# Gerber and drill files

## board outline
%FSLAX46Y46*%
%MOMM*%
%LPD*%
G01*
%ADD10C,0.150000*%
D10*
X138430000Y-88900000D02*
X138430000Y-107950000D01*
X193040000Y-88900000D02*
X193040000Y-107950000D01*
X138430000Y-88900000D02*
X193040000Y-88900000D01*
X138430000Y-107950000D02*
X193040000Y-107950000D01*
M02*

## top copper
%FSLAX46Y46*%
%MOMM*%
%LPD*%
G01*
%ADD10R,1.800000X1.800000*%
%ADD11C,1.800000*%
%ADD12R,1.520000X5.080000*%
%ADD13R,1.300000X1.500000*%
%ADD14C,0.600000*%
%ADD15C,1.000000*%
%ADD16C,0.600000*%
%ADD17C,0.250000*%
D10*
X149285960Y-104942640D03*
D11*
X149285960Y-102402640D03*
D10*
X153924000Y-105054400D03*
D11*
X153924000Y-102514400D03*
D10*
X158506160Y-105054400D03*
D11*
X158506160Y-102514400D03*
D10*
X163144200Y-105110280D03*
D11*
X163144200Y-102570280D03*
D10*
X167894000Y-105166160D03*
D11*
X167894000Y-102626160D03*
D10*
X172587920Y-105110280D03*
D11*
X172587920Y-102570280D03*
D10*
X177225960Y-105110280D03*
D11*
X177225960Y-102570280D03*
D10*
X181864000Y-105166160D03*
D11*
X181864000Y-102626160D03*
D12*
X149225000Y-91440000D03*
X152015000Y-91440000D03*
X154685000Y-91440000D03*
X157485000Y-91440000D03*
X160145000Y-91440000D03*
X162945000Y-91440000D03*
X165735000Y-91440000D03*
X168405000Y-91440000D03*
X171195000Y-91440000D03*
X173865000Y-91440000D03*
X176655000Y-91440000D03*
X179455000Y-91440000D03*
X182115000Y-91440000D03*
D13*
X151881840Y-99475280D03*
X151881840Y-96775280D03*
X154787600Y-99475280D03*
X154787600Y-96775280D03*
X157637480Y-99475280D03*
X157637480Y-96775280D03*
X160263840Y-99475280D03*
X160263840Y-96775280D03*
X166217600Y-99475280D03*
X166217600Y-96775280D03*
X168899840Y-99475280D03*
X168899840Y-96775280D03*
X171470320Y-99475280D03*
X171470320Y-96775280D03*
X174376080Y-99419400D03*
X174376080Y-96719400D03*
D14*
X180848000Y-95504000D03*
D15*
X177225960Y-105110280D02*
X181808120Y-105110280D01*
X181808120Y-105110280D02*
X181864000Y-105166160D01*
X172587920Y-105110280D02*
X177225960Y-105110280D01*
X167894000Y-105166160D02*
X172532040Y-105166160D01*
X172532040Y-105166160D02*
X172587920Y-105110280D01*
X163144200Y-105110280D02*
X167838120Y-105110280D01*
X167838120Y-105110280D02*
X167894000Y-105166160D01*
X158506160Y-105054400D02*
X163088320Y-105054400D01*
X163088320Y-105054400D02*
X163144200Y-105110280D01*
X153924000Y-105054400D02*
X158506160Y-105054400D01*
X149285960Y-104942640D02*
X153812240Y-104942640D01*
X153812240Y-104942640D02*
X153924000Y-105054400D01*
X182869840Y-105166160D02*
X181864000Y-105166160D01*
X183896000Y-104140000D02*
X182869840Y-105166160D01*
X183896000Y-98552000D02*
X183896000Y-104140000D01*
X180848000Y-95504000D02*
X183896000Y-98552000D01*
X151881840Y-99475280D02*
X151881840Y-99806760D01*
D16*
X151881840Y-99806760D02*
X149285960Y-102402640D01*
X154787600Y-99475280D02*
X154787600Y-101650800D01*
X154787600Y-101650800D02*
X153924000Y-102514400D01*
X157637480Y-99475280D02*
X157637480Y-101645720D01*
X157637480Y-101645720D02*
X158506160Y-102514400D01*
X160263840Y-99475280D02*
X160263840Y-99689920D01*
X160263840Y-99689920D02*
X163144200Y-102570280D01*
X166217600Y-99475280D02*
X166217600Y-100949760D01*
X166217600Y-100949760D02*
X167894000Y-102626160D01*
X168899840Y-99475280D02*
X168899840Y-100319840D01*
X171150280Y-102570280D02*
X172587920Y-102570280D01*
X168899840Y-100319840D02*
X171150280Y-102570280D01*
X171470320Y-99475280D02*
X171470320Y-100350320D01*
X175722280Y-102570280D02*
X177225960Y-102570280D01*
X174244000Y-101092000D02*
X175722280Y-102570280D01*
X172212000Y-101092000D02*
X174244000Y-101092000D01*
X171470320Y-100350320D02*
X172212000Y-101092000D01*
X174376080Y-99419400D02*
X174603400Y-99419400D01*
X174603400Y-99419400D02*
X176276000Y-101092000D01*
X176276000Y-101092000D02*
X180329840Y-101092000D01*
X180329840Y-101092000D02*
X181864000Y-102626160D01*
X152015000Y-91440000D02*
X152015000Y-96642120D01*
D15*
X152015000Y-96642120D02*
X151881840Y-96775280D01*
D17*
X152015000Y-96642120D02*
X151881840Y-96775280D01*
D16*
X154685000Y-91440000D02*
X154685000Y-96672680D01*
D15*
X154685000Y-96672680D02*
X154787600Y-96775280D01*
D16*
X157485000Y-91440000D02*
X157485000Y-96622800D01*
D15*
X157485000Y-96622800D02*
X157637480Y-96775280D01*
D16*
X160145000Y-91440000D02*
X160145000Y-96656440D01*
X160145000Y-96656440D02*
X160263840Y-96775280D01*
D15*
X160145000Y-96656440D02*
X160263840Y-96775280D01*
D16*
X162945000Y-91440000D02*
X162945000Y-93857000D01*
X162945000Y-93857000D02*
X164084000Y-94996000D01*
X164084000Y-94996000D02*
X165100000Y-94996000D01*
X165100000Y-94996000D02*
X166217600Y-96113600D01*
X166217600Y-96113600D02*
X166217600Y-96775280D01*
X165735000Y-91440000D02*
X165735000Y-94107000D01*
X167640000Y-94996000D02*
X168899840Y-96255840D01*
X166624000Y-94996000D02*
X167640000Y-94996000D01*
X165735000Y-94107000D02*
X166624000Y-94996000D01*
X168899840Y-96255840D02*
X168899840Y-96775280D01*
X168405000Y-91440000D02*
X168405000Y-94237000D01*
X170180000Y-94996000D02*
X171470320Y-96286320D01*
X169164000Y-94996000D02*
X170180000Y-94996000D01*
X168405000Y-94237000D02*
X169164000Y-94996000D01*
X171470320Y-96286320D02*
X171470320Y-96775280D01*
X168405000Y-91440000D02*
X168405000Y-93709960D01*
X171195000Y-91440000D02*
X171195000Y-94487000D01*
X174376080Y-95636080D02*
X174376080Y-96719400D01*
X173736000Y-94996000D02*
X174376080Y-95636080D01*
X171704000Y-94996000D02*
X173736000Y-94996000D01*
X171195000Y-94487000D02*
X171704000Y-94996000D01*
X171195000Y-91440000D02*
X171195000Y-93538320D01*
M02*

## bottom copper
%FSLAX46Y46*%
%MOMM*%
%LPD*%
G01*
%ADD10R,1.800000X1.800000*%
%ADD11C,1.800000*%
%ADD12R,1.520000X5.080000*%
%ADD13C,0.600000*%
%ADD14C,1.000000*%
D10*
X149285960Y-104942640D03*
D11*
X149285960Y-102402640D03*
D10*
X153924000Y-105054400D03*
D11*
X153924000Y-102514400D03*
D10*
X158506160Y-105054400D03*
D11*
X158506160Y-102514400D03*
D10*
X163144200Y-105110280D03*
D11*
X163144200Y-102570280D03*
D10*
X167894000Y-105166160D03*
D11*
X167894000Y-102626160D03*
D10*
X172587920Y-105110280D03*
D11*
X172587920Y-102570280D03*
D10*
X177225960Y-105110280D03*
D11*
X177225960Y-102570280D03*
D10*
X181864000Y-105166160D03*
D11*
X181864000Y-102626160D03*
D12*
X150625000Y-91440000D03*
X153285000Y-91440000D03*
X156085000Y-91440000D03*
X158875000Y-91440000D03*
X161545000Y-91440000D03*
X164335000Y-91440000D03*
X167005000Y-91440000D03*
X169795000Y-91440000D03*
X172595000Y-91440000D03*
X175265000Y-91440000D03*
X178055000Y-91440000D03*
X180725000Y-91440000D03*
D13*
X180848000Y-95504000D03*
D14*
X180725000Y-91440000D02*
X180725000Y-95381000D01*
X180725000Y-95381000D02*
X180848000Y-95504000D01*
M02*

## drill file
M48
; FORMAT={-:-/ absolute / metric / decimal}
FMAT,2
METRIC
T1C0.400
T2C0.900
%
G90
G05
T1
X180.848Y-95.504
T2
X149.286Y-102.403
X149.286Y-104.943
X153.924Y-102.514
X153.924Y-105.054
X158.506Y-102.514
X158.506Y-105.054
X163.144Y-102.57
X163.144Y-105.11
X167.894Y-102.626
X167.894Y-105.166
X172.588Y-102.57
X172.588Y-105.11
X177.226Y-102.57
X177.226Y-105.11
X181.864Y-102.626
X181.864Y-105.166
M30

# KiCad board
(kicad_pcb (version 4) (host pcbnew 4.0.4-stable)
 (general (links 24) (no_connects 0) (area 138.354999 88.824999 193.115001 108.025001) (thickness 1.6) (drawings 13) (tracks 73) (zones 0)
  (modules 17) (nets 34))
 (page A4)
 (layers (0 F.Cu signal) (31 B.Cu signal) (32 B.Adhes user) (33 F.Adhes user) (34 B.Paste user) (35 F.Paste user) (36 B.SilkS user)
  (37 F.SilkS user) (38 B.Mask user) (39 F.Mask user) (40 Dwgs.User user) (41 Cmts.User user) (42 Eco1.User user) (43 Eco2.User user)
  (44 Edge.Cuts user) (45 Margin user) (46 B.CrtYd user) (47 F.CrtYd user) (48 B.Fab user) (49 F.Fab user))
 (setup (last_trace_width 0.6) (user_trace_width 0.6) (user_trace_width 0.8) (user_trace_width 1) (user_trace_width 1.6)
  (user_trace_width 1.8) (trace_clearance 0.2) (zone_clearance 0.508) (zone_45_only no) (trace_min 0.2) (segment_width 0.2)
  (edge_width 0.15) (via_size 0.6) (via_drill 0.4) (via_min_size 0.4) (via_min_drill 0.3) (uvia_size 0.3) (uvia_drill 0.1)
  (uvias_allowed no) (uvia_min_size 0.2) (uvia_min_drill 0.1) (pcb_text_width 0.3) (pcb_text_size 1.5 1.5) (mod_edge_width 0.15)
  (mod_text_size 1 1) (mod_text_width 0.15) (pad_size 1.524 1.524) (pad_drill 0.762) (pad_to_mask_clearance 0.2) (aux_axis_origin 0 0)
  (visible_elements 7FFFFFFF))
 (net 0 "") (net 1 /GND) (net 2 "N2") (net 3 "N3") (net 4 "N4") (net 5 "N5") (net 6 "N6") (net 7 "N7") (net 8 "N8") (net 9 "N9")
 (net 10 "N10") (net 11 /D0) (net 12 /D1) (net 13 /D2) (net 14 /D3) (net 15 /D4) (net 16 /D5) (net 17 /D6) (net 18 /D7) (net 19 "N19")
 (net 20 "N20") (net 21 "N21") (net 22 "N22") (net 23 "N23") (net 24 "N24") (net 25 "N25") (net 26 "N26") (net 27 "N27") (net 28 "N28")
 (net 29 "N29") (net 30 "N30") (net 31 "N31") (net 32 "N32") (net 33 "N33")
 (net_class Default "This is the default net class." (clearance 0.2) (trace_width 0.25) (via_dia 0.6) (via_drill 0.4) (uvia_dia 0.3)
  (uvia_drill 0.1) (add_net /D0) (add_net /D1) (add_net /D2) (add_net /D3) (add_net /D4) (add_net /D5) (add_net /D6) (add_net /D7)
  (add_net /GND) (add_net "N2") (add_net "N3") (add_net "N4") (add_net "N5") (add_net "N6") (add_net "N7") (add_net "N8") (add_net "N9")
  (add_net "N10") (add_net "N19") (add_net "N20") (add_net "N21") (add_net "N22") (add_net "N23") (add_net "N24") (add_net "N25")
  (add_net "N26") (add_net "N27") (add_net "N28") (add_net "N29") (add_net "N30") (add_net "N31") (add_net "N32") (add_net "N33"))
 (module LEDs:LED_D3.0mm (layer F.Cu) (at 149.28596 104.94264 90)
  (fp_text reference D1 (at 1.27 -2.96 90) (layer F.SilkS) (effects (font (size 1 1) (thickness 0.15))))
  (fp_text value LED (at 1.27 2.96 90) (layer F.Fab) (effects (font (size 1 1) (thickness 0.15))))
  (pad 1 thru_hole rect (at 0 0 90) (size 1.8 1.8) (drill 0.9) (layers *.Cu *.Mask) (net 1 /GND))
  (pad 2 thru_hole circle (at 2.54 0 90) (size 1.8 1.8) (drill 0.9) (layers *.Cu *.Mask) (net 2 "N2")))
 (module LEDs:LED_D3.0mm (layer F.Cu) (at 153.924 105.0544 90)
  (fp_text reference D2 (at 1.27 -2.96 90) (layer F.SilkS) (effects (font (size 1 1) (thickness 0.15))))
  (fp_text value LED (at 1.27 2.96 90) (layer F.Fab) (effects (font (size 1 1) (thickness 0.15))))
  (pad 1 thru_hole rect (at 0 0 90) (size 1.8 1.8) (drill 0.9) (layers *.Cu *.Mask) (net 1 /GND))
  (pad 2 thru_hole circle (at 2.54 0 90) (size 1.8 1.8) (drill 0.9) (layers *.Cu *.Mask) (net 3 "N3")))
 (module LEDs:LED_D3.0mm (layer F.Cu) (at 158.50616 105.0544 90)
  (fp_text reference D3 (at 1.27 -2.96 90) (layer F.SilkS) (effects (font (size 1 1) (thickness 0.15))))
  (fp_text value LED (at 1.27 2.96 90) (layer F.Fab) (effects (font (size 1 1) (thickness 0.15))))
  (pad 1 thru_hole rect (at 0 0 90) (size 1.8 1.8) (drill 0.9) (layers *.Cu *.Mask) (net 1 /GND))
  (pad 2 thru_hole circle (at 2.54 0 90) (size 1.8 1.8) (drill 0.9) (layers *.Cu *.Mask) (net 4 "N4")))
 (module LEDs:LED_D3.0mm (layer F.Cu) (at 163.1442 105.11028 90)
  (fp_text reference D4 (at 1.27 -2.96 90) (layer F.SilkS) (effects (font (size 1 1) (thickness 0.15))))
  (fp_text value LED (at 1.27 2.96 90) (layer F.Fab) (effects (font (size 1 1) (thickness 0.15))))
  (pad 1 thru_hole rect (at 0 0 90) (size 1.8 1.8) (drill 0.9) (layers *.Cu *.Mask) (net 1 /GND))
  (pad 2 thru_hole circle (at 2.54 0 90) (size 1.8 1.8) (drill 0.9) (layers *.Cu *.Mask) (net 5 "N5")))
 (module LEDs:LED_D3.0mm (layer F.Cu) (at 167.894 105.16616 90)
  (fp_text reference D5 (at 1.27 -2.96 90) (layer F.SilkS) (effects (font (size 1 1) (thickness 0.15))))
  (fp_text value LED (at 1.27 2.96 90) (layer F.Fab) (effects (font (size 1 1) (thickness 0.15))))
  (pad 1 thru_hole rect (at 0 0 90) (size 1.8 1.8) (drill 0.9) (layers *.Cu *.Mask) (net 1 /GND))
  (pad 2 thru_hole circle (at 2.54 0 90) (size 1.8 1.8) (drill 0.9) (layers *.Cu *.Mask) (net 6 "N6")))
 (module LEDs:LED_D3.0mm (layer F.Cu) (at 172.58792 105.11028 90)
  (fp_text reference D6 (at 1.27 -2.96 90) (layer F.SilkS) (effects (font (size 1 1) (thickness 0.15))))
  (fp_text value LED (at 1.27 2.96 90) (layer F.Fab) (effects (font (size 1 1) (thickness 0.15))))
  (pad 1 thru_hole rect (at 0 0 90) (size 1.8 1.8) (drill 0.9) (layers *.Cu *.Mask) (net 1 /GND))
  (pad 2 thru_hole circle (at 2.54 0 90) (size 1.8 1.8) (drill 0.9) (layers *.Cu *.Mask) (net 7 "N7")))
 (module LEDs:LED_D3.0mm (layer F.Cu) (at 177.22596 105.11028 90)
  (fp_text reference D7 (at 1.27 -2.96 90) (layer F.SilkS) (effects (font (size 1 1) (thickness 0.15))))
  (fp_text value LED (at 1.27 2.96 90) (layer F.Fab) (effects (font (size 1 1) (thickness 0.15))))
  (pad 1 thru_hole rect (at 0 0 90) (size 1.8 1.8) (drill 0.9) (layers *.Cu *.Mask) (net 1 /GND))
  (pad 2 thru_hole circle (at 2.54 0 90) (size 1.8 1.8) (drill 0.9) (layers *.Cu *.Mask) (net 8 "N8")))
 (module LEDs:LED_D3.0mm (layer F.Cu) (at 181.864 105.16616 90)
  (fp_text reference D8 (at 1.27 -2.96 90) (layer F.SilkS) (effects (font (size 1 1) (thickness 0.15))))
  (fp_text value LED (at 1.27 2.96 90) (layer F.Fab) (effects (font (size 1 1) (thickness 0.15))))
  (pad 1 thru_hole rect (at 0 0 90) (size 1.8 1.8) (drill 0.9) (layers *.Cu *.Mask) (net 1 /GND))
  (pad 2 thru_hole circle (at 2.54 0 90) (size 1.8 1.8) (drill 0.9) (layers *.Cu *.Mask) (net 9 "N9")))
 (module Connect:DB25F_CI (layer F.Cu) (at 149.225 91.44)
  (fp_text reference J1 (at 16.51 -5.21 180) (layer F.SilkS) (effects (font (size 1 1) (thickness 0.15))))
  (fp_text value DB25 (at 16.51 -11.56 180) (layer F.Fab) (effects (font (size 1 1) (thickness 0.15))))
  (pad 1 connect rect (at 0 0 90) (size 5.08 1.52) (layers F.Cu F.Mask) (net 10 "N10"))
  (pad 2 connect rect (at 2.79 0 90) (size 5.08 1.52) (layers F.Cu F.Mask) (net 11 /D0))
  (pad 3 connect rect (at 5.46 0 90) (size 5.08 1.52) (layers F.Cu F.Mask) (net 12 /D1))
  (pad 4 connect rect (at 8.26 0 90) (size 5.08 1.52) (layers F.Cu F.Mask) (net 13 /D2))
  (pad 5 connect rect (at 10.92 0 90) (size 5.08 1.52) (layers F.Cu F.Mask) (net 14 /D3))
  (pad 6 connect rect (at 13.72 0 90) (size 5.08 1.52) (layers F.Cu F.Mask) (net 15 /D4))
  (pad 7 connect rect (at 16.51 0 90) (size 5.08 1.52) (layers F.Cu F.Mask) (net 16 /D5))
  (pad 8 connect rect (at 19.18 0 90) (size 5.08 1.52) (layers F.Cu F.Mask) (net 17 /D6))
  (pad 9 connect rect (at 21.97 0 90) (size 5.08 1.52) (layers F.Cu F.Mask) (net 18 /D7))
  (pad 10 connect rect (at 24.64 0 90) (size 5.08 1.52) (layers F.Cu F.Mask) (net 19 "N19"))
  (pad 11 connect rect (at 27.43 0 90) (size 5.08 1.52) (layers F.Cu F.Mask) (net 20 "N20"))
  (pad 12 connect rect (at 30.23 0 90) (size 5.08 1.52) (layers F.Cu F.Mask) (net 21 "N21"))
  (pad 13 connect rect (at 32.89 0 90) (size 5.08 1.52) (layers F.Cu F.Mask) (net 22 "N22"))
  (pad 14 connect rect (at 1.4 0 90) (size 5.08 1.52) (layers B.Cu B.Mask) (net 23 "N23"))
  (pad 15 connect rect (at 4.06 0 90) (size 5.08 1.52) (layers B.Cu B.Mask) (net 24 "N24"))
  (pad 16 connect rect (at 6.86 0 90) (size 5.08 1.52) (layers B.Cu B.Mask) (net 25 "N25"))
  (pad 17 connect rect (at 9.65 0 90) (size 5.08 1.52) (layers B.Cu B.Mask) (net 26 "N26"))
  (pad 18 connect rect (at 12.32 0 90) (size 5.08 1.52) (layers B.Cu B.Mask) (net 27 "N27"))
  (pad 19 connect rect (at 15.11 0 90) (size 5.08 1.52) (layers B.Cu B.Mask) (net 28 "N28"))
  (pad 20 connect rect (at 17.78 0 90) (size 5.08 1.52) (layers B.Cu B.Mask) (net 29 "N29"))
  (pad 21 connect rect (at 20.57 0 90) (size 5.08 1.52) (layers B.Cu B.Mask) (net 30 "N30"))
  (pad 22 connect rect (at 23.37 0 90) (size 5.08 1.52) (layers B.Cu B.Mask) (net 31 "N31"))
  (pad 23 connect rect (at 26.04 0 90) (size 5.08 1.52) (layers B.Cu B.Mask) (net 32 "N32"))
  (pad 24 connect rect (at 28.83 0 90) (size 5.08 1.52) (layers B.Cu B.Mask) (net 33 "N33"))
  (pad 25 connect rect (at 31.5 0 90) (size 5.08 1.52) (layers B.Cu B.Mask) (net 1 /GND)))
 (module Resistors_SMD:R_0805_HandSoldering (layer F.Cu) (at 151.88184 98.12528 90)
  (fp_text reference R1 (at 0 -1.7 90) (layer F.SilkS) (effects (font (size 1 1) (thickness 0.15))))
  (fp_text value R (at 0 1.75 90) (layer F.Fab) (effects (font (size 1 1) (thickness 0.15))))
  (pad 1 smd rect (at -1.35 0 90) (size 1.5 1.3) (layers F.Cu F.Paste F.Mask) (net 2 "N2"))
  (pad 2 smd rect (at 1.35 0 90) (size 1.5 1.3) (layers F.Cu F.Paste F.Mask) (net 11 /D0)))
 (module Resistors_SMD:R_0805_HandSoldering (layer F.Cu) (at 154.7876 98.12528 90)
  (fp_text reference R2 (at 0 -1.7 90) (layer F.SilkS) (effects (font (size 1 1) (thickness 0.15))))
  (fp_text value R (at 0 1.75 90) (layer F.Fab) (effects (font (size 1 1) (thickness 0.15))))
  (pad 1 smd rect (at -1.35 0 90) (size 1.5 1.3) (layers F.Cu F.Paste F.Mask) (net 3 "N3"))
  (pad 2 smd rect (at 1.35 0 90) (size 1.5 1.3) (layers F.Cu F.Paste F.Mask) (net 12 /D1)))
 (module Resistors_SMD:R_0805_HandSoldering (layer F.Cu) (at 157.63748 98.12528 90)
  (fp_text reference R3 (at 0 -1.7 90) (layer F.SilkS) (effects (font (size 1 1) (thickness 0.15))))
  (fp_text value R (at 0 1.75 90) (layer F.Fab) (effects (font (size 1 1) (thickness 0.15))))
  (pad 1 smd rect (at -1.35 0 90) (size 1.5 1.3) (layers F.Cu F.Paste F.Mask) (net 4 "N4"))
  (pad 2 smd rect (at 1.35 0 90) (size 1.5 1.3) (layers F.Cu F.Paste F.Mask) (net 13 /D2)))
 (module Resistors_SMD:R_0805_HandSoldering (layer F.Cu) (at 160.26384 98.12528 90)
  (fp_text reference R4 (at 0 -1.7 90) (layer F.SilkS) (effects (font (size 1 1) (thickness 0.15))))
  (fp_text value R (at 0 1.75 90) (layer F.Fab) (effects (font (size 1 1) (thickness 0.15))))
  (pad 1 smd rect (at -1.35 0 90) (size 1.5 1.3) (layers F.Cu F.Paste F.Mask) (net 5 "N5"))
  (pad 2 smd rect (at 1.35 0 90) (size 1.5 1.3) (layers F.Cu F.Paste F.Mask) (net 14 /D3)))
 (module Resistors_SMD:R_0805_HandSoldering (layer F.Cu) (at 166.2176 98.12528 90)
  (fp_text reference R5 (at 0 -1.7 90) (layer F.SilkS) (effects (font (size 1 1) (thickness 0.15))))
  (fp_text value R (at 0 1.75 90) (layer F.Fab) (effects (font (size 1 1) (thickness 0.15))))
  (pad 1 smd rect (at -1.35 0 90) (size 1.5 1.3) (layers F.Cu F.Paste F.Mask) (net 6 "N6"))
  (pad 2 smd rect (at 1.35 0 90) (size 1.5 1.3) (layers F.Cu F.Paste F.Mask) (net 15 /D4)))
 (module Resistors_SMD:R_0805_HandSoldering (layer F.Cu) (at 168.89984 98.12528 90)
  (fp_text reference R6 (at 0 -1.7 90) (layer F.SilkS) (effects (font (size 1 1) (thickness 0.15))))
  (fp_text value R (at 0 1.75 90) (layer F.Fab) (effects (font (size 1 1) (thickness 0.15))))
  (pad 1 smd rect (at -1.35 0 90) (size 1.5 1.3) (layers F.Cu F.Paste F.Mask) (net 7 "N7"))
  (pad 2 smd rect (at 1.35 0 90) (size 1.5 1.3) (layers F.Cu F.Paste F.Mask) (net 16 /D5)))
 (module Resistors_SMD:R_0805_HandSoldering (layer F.Cu) (at 171.47032 98.12528 90)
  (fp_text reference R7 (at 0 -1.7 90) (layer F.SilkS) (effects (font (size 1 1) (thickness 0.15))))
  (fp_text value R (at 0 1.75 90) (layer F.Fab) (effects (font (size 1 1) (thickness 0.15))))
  (pad 1 smd rect (at -1.35 0 90) (size 1.5 1.3) (layers F.Cu F.Paste F.Mask) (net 8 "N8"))
  (pad 2 smd rect (at 1.35 0 90) (size 1.5 1.3) (layers F.Cu F.Paste F.Mask) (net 17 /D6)))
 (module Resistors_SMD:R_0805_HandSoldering (layer F.Cu) (at 174.37608 98.0694 90)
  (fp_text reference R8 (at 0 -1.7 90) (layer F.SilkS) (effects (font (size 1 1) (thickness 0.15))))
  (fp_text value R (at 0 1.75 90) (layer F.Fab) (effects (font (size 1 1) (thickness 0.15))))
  (pad 1 smd rect (at -1.35 0 90) (size 1.5 1.3) (layers F.Cu F.Paste F.Mask) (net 9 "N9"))
  (pad 2 smd rect (at 1.35 0 90) (size 1.5 1.3) (layers F.Cu F.Paste F.Mask) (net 18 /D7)))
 (gr_line (start 138.43 88.9) (end 138.43 107.95) (angle 90) (layer Edge.Cuts) (width 0.15))
 (gr_line (start 193.04 88.9) (end 193.04 107.95) (angle 90) (layer Edge.Cuts) (width 0.15))
 (gr_line (start 138.43 88.9) (end 193.04 88.9) (angle 90) (layer Edge.Cuts) (width 0.15))
 (gr_line (start 138.43 107.95) (end 193.04 107.95) (angle 90) (layer Edge.Cuts) (width 0.15))
 (segment (start 177.22596 105.11028) (end 181.80812 105.11028) (width 1) (layer F.Cu) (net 1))
 (segment (start 181.80812 105.11028) (end 181.864 105.16616) (width 1) (layer F.Cu) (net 1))
 (segment (start 172.58792 105.11028) (end 177.22596 105.11028) (width 1) (layer F.Cu) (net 1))
 (segment (start 167.894 105.16616) (end 172.53204 105.16616) (width 1) (layer F.Cu) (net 1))
 (segment (start 172.53204 105.16616) (end 172.58792 105.11028) (width 1) (layer F.Cu) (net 1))
 (segment (start 163.1442 105.11028) (end 167.83812 105.11028) (width 1) (layer F.Cu) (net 1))
 (segment (start 167.83812 105.11028) (end 167.894 105.16616) (width 1) (layer F.Cu) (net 1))
 (segment (start 158.50616 105.0544) (end 163.08832 105.0544) (width 1) (layer F.Cu) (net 1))
 (segment (start 163.08832 105.0544) (end 163.1442 105.11028) (width 1) (layer F.Cu) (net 1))
 (segment (start 153.924 105.0544) (end 158.50616 105.0544) (width 1) (layer F.Cu) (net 1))
 (segment (start 149.28596 104.94264) (end 153.81224 104.94264) (width 1) (layer F.Cu) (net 1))
 (segment (start 153.81224 104.94264) (end 153.924 105.0544) (width 1) (layer F.Cu) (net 1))
 (segment (start 180.725 91.44) (end 180.725 95.381) (width 1) (layer B.Cu) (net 1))
 (segment (start 182.86984 105.16616) (end 181.864 105.16616) (width 1) (layer F.Cu) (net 1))
 (segment (start 183.896 104.14) (end 182.86984 105.16616) (width 1) (layer F.Cu) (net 1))
 (segment (start 183.896 98.552) (end 183.896 104.14) (width 1) (layer F.Cu) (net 1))
 (segment (start 180.848 95.504) (end 183.896 98.552) (width 1) (layer F.Cu) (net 1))
 (via (at 180.848 95.504) (size 0.6) (drill 0.4) (layers F.Cu B.Cu) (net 1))
 (segment (start 180.725 95.381) (end 180.848 95.504) (width 1) (layer B.Cu) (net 1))
 (segment (start 151.88184 99.47528) (end 151.88184 99.80676) (width 1) (layer F.Cu) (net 2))
 (segment (start 151.88184 99.80676) (end 149.28596 102.40264) (width 0.6) (layer F.Cu) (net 2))
 (segment (start 154.7876 99.47528) (end 154.7876 101.6508) (width 0.6) (layer F.Cu) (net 3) (status 400000))
 (segment (start 154.7876 101.6508) (end 153.924 102.5144) (width 0.6) (layer F.Cu) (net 3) (status 800000))
 (segment (start 157.63748 99.47528) (end 157.63748 101.64572) (width 0.6) (layer F.Cu) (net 4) (status 400000))
 (segment (start 157.63748 101.64572) (end 158.50616 102.5144) (width 0.6) (layer F.Cu) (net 4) (status 800000))
 (segment (start 160.26384 99.47528) (end 160.26384 99.68992) (width 0.6) (layer F.Cu) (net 5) (status C00000))
 (segment (start 160.26384 99.68992) (end 163.1442 102.57028) (width 0.6) (layer F.Cu) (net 5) (status C00000))
 (segment (start 166.2176 99.47528) (end 166.2176 100.94976) (width 0.6) (layer F.Cu) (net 6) (status 400000))
 (segment (start 166.2176 100.94976) (end 167.894 102.62616) (width 0.6) (layer F.Cu) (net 6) (status 800000))
 (segment (start 168.89984 99.47528) (end 168.89984 100.31984) (width 0.6) (layer F.Cu) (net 7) (status 400000))
 (segment (start 171.15028 102.57028) (end 172.58792 102.57028) (width 0.6) (layer F.Cu) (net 7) (status 800000))
 (segment (start 168.89984 100.31984) (end 171.15028 102.57028) (width 0.6) (layer F.Cu) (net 7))
 (segment (start 171.47032 99.47528) (end 171.47032 100.35032) (width 0.6) (layer F.Cu) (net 8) (status 400000))
 (segment (start 175.72228 102.57028) (end 177.22596 102.57028) (width 0.6) (layer F.Cu) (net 8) (status 800000))
 (segment (start 174.244 101.092) (end 175.72228 102.57028) (width 0.6) (layer F.Cu) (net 8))
 (segment (start 172.212 101.092) (end 174.244 101.092) (width 0.6) (layer F.Cu) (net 8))
 (segment (start 171.47032 100.35032) (end 172.212 101.092) (width 0.6) (layer F.Cu) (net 8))
 (segment (start 174.37608 99.4194) (end 174.6034 99.4194) (width 0.6) (layer F.Cu) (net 9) (status C00000))
 (segment (start 174.6034 99.4194) (end 176.276 101.092) (width 0.6) (layer F.Cu) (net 9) (status 400000))
 (segment (start 176.276 101.092) (end 180.32984 101.092) (width 0.6) (layer F.Cu) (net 9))
 (segment (start 180.32984 101.092) (end 181.864 102.62616) (width 0.6) (layer F.Cu) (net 9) (status 800000))
 (segment (start 152.015 91.44) (end 152.015 96.64212) (width 0.6) (layer F.Cu) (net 11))
 (segment (start 152.015 96.64212) (end 151.88184 96.77528) (width 1) (layer F.Cu) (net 11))
 (segment (start 152.015 96.64212) (end 151.88184 96.77528) (width 0.25) (layer F.Cu) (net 11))
 (segment (start 154.685 91.44) (end 154.685 96.67268) (width 0.6) (layer F.Cu) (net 12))
 (segment (start 154.685 96.67268) (end 154.7876 96.77528) (width 1) (layer F.Cu) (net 12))
 (segment (start 157.485 91.44) (end 157.485 96.6228) (width 0.6) (layer F.Cu) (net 13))
 (segment (start 157.485 96.6228) (end 157.63748 96.77528) (width 1) (layer F.Cu) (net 13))
 (segment (start 160.145 91.44) (end 160.145 96.65644) (width 0.6) (layer F.Cu) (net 14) (status C00000))
 (segment (start 160.145 96.65644) (end 160.26384 96.77528) (width 0.6) (layer F.Cu) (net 14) (status C00000))
 (segment (start 160.145 96.65644) (end 160.26384 96.77528) (width 1) (layer F.Cu) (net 14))
 (segment (start 162.945 91.44) (end 162.945 93.857) (width 0.6) (layer F.Cu) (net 15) (status C00000))
 (segment (start 162.945 93.857) (end 164.084 94.996) (width 0.6) (layer F.Cu) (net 15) (status 400000))
 (segment (start 164.084 94.996) (end 165.1 94.996) (width 0.6) (layer F.Cu) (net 15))
 (segment (start 165.1 94.996) (end 166.2176 96.1136) (width 0.6) (layer F.Cu) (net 15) (status 800000))
 (segment (start 166.2176 96.1136) (end 166.2176 96.77528) (width 0.6) (layer F.Cu) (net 15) (status C00000))
 (segment (start 165.735 91.44) (end 165.735 94.107) (width 0.6) (layer F.Cu) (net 16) (status 400000))
 (segment (start 167.64 94.996) (end 168.89984 96.25584) (width 0.6) (layer F.Cu) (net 16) (status 800000))
 (segment (start 166.624 94.996) (end 167.64 94.996) (width 0.6) (layer F.Cu) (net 16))
 (segment (start 165.735 94.107) (end 166.624 94.996) (width 0.6) (layer F.Cu) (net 16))
 (segment (start 168.89984 96.25584) (end 168.89984 96.77528) (width 0.6) (layer F.Cu) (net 16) (status C00000))
 (segment (start 168.405 91.44) (end 168.405 94.237) (width 0.6) (layer F.Cu) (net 17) (status 400000))
 (segment (start 170.18 94.996) (end 171.47032 96.28632) (width 0.6) (layer F.Cu) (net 17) (status 800000))
 (segment (start 169.164 94.996) (end 170.18 94.996) (width 0.6) (layer F.Cu) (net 17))
 (segment (start 168.405 94.237) (end 169.164 94.996) (width 0.6) (layer F.Cu) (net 17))
 (segment (start 171.47032 96.28632) (end 171.47032 96.77528) (width 0.6) (layer F.Cu) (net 17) (status C00000))
 (segment (start 168.405 91.44) (end 168.405 93.70996) (width 0.6) (layer F.Cu) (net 17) (status C00000))
 (segment (start 171.195 91.44) (end 171.195 94.487) (width 0.6) (layer F.Cu) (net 18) (status 400000))
 (segment (start 174.37608 95.63608) (end 174.37608 96.7194) (width 0.6) (layer F.Cu) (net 18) (status 800000))
 (segment (start 173.736 94.996) (end 174.37608 95.63608) (width 0.6) (layer F.Cu) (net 18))
 (segment (start 171.704 94.996) (end 173.736 94.996) (width 0.6) (layer F.Cu) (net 18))
 (segment (start 171.195 94.487) (end 171.704 94.996) (width 0.6) (layer F.Cu) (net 18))
 (segment (start 171.195 91.44) (end 171.195 93.53832) (width 0.6) (layer F.Cu) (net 18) (status C00000)))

